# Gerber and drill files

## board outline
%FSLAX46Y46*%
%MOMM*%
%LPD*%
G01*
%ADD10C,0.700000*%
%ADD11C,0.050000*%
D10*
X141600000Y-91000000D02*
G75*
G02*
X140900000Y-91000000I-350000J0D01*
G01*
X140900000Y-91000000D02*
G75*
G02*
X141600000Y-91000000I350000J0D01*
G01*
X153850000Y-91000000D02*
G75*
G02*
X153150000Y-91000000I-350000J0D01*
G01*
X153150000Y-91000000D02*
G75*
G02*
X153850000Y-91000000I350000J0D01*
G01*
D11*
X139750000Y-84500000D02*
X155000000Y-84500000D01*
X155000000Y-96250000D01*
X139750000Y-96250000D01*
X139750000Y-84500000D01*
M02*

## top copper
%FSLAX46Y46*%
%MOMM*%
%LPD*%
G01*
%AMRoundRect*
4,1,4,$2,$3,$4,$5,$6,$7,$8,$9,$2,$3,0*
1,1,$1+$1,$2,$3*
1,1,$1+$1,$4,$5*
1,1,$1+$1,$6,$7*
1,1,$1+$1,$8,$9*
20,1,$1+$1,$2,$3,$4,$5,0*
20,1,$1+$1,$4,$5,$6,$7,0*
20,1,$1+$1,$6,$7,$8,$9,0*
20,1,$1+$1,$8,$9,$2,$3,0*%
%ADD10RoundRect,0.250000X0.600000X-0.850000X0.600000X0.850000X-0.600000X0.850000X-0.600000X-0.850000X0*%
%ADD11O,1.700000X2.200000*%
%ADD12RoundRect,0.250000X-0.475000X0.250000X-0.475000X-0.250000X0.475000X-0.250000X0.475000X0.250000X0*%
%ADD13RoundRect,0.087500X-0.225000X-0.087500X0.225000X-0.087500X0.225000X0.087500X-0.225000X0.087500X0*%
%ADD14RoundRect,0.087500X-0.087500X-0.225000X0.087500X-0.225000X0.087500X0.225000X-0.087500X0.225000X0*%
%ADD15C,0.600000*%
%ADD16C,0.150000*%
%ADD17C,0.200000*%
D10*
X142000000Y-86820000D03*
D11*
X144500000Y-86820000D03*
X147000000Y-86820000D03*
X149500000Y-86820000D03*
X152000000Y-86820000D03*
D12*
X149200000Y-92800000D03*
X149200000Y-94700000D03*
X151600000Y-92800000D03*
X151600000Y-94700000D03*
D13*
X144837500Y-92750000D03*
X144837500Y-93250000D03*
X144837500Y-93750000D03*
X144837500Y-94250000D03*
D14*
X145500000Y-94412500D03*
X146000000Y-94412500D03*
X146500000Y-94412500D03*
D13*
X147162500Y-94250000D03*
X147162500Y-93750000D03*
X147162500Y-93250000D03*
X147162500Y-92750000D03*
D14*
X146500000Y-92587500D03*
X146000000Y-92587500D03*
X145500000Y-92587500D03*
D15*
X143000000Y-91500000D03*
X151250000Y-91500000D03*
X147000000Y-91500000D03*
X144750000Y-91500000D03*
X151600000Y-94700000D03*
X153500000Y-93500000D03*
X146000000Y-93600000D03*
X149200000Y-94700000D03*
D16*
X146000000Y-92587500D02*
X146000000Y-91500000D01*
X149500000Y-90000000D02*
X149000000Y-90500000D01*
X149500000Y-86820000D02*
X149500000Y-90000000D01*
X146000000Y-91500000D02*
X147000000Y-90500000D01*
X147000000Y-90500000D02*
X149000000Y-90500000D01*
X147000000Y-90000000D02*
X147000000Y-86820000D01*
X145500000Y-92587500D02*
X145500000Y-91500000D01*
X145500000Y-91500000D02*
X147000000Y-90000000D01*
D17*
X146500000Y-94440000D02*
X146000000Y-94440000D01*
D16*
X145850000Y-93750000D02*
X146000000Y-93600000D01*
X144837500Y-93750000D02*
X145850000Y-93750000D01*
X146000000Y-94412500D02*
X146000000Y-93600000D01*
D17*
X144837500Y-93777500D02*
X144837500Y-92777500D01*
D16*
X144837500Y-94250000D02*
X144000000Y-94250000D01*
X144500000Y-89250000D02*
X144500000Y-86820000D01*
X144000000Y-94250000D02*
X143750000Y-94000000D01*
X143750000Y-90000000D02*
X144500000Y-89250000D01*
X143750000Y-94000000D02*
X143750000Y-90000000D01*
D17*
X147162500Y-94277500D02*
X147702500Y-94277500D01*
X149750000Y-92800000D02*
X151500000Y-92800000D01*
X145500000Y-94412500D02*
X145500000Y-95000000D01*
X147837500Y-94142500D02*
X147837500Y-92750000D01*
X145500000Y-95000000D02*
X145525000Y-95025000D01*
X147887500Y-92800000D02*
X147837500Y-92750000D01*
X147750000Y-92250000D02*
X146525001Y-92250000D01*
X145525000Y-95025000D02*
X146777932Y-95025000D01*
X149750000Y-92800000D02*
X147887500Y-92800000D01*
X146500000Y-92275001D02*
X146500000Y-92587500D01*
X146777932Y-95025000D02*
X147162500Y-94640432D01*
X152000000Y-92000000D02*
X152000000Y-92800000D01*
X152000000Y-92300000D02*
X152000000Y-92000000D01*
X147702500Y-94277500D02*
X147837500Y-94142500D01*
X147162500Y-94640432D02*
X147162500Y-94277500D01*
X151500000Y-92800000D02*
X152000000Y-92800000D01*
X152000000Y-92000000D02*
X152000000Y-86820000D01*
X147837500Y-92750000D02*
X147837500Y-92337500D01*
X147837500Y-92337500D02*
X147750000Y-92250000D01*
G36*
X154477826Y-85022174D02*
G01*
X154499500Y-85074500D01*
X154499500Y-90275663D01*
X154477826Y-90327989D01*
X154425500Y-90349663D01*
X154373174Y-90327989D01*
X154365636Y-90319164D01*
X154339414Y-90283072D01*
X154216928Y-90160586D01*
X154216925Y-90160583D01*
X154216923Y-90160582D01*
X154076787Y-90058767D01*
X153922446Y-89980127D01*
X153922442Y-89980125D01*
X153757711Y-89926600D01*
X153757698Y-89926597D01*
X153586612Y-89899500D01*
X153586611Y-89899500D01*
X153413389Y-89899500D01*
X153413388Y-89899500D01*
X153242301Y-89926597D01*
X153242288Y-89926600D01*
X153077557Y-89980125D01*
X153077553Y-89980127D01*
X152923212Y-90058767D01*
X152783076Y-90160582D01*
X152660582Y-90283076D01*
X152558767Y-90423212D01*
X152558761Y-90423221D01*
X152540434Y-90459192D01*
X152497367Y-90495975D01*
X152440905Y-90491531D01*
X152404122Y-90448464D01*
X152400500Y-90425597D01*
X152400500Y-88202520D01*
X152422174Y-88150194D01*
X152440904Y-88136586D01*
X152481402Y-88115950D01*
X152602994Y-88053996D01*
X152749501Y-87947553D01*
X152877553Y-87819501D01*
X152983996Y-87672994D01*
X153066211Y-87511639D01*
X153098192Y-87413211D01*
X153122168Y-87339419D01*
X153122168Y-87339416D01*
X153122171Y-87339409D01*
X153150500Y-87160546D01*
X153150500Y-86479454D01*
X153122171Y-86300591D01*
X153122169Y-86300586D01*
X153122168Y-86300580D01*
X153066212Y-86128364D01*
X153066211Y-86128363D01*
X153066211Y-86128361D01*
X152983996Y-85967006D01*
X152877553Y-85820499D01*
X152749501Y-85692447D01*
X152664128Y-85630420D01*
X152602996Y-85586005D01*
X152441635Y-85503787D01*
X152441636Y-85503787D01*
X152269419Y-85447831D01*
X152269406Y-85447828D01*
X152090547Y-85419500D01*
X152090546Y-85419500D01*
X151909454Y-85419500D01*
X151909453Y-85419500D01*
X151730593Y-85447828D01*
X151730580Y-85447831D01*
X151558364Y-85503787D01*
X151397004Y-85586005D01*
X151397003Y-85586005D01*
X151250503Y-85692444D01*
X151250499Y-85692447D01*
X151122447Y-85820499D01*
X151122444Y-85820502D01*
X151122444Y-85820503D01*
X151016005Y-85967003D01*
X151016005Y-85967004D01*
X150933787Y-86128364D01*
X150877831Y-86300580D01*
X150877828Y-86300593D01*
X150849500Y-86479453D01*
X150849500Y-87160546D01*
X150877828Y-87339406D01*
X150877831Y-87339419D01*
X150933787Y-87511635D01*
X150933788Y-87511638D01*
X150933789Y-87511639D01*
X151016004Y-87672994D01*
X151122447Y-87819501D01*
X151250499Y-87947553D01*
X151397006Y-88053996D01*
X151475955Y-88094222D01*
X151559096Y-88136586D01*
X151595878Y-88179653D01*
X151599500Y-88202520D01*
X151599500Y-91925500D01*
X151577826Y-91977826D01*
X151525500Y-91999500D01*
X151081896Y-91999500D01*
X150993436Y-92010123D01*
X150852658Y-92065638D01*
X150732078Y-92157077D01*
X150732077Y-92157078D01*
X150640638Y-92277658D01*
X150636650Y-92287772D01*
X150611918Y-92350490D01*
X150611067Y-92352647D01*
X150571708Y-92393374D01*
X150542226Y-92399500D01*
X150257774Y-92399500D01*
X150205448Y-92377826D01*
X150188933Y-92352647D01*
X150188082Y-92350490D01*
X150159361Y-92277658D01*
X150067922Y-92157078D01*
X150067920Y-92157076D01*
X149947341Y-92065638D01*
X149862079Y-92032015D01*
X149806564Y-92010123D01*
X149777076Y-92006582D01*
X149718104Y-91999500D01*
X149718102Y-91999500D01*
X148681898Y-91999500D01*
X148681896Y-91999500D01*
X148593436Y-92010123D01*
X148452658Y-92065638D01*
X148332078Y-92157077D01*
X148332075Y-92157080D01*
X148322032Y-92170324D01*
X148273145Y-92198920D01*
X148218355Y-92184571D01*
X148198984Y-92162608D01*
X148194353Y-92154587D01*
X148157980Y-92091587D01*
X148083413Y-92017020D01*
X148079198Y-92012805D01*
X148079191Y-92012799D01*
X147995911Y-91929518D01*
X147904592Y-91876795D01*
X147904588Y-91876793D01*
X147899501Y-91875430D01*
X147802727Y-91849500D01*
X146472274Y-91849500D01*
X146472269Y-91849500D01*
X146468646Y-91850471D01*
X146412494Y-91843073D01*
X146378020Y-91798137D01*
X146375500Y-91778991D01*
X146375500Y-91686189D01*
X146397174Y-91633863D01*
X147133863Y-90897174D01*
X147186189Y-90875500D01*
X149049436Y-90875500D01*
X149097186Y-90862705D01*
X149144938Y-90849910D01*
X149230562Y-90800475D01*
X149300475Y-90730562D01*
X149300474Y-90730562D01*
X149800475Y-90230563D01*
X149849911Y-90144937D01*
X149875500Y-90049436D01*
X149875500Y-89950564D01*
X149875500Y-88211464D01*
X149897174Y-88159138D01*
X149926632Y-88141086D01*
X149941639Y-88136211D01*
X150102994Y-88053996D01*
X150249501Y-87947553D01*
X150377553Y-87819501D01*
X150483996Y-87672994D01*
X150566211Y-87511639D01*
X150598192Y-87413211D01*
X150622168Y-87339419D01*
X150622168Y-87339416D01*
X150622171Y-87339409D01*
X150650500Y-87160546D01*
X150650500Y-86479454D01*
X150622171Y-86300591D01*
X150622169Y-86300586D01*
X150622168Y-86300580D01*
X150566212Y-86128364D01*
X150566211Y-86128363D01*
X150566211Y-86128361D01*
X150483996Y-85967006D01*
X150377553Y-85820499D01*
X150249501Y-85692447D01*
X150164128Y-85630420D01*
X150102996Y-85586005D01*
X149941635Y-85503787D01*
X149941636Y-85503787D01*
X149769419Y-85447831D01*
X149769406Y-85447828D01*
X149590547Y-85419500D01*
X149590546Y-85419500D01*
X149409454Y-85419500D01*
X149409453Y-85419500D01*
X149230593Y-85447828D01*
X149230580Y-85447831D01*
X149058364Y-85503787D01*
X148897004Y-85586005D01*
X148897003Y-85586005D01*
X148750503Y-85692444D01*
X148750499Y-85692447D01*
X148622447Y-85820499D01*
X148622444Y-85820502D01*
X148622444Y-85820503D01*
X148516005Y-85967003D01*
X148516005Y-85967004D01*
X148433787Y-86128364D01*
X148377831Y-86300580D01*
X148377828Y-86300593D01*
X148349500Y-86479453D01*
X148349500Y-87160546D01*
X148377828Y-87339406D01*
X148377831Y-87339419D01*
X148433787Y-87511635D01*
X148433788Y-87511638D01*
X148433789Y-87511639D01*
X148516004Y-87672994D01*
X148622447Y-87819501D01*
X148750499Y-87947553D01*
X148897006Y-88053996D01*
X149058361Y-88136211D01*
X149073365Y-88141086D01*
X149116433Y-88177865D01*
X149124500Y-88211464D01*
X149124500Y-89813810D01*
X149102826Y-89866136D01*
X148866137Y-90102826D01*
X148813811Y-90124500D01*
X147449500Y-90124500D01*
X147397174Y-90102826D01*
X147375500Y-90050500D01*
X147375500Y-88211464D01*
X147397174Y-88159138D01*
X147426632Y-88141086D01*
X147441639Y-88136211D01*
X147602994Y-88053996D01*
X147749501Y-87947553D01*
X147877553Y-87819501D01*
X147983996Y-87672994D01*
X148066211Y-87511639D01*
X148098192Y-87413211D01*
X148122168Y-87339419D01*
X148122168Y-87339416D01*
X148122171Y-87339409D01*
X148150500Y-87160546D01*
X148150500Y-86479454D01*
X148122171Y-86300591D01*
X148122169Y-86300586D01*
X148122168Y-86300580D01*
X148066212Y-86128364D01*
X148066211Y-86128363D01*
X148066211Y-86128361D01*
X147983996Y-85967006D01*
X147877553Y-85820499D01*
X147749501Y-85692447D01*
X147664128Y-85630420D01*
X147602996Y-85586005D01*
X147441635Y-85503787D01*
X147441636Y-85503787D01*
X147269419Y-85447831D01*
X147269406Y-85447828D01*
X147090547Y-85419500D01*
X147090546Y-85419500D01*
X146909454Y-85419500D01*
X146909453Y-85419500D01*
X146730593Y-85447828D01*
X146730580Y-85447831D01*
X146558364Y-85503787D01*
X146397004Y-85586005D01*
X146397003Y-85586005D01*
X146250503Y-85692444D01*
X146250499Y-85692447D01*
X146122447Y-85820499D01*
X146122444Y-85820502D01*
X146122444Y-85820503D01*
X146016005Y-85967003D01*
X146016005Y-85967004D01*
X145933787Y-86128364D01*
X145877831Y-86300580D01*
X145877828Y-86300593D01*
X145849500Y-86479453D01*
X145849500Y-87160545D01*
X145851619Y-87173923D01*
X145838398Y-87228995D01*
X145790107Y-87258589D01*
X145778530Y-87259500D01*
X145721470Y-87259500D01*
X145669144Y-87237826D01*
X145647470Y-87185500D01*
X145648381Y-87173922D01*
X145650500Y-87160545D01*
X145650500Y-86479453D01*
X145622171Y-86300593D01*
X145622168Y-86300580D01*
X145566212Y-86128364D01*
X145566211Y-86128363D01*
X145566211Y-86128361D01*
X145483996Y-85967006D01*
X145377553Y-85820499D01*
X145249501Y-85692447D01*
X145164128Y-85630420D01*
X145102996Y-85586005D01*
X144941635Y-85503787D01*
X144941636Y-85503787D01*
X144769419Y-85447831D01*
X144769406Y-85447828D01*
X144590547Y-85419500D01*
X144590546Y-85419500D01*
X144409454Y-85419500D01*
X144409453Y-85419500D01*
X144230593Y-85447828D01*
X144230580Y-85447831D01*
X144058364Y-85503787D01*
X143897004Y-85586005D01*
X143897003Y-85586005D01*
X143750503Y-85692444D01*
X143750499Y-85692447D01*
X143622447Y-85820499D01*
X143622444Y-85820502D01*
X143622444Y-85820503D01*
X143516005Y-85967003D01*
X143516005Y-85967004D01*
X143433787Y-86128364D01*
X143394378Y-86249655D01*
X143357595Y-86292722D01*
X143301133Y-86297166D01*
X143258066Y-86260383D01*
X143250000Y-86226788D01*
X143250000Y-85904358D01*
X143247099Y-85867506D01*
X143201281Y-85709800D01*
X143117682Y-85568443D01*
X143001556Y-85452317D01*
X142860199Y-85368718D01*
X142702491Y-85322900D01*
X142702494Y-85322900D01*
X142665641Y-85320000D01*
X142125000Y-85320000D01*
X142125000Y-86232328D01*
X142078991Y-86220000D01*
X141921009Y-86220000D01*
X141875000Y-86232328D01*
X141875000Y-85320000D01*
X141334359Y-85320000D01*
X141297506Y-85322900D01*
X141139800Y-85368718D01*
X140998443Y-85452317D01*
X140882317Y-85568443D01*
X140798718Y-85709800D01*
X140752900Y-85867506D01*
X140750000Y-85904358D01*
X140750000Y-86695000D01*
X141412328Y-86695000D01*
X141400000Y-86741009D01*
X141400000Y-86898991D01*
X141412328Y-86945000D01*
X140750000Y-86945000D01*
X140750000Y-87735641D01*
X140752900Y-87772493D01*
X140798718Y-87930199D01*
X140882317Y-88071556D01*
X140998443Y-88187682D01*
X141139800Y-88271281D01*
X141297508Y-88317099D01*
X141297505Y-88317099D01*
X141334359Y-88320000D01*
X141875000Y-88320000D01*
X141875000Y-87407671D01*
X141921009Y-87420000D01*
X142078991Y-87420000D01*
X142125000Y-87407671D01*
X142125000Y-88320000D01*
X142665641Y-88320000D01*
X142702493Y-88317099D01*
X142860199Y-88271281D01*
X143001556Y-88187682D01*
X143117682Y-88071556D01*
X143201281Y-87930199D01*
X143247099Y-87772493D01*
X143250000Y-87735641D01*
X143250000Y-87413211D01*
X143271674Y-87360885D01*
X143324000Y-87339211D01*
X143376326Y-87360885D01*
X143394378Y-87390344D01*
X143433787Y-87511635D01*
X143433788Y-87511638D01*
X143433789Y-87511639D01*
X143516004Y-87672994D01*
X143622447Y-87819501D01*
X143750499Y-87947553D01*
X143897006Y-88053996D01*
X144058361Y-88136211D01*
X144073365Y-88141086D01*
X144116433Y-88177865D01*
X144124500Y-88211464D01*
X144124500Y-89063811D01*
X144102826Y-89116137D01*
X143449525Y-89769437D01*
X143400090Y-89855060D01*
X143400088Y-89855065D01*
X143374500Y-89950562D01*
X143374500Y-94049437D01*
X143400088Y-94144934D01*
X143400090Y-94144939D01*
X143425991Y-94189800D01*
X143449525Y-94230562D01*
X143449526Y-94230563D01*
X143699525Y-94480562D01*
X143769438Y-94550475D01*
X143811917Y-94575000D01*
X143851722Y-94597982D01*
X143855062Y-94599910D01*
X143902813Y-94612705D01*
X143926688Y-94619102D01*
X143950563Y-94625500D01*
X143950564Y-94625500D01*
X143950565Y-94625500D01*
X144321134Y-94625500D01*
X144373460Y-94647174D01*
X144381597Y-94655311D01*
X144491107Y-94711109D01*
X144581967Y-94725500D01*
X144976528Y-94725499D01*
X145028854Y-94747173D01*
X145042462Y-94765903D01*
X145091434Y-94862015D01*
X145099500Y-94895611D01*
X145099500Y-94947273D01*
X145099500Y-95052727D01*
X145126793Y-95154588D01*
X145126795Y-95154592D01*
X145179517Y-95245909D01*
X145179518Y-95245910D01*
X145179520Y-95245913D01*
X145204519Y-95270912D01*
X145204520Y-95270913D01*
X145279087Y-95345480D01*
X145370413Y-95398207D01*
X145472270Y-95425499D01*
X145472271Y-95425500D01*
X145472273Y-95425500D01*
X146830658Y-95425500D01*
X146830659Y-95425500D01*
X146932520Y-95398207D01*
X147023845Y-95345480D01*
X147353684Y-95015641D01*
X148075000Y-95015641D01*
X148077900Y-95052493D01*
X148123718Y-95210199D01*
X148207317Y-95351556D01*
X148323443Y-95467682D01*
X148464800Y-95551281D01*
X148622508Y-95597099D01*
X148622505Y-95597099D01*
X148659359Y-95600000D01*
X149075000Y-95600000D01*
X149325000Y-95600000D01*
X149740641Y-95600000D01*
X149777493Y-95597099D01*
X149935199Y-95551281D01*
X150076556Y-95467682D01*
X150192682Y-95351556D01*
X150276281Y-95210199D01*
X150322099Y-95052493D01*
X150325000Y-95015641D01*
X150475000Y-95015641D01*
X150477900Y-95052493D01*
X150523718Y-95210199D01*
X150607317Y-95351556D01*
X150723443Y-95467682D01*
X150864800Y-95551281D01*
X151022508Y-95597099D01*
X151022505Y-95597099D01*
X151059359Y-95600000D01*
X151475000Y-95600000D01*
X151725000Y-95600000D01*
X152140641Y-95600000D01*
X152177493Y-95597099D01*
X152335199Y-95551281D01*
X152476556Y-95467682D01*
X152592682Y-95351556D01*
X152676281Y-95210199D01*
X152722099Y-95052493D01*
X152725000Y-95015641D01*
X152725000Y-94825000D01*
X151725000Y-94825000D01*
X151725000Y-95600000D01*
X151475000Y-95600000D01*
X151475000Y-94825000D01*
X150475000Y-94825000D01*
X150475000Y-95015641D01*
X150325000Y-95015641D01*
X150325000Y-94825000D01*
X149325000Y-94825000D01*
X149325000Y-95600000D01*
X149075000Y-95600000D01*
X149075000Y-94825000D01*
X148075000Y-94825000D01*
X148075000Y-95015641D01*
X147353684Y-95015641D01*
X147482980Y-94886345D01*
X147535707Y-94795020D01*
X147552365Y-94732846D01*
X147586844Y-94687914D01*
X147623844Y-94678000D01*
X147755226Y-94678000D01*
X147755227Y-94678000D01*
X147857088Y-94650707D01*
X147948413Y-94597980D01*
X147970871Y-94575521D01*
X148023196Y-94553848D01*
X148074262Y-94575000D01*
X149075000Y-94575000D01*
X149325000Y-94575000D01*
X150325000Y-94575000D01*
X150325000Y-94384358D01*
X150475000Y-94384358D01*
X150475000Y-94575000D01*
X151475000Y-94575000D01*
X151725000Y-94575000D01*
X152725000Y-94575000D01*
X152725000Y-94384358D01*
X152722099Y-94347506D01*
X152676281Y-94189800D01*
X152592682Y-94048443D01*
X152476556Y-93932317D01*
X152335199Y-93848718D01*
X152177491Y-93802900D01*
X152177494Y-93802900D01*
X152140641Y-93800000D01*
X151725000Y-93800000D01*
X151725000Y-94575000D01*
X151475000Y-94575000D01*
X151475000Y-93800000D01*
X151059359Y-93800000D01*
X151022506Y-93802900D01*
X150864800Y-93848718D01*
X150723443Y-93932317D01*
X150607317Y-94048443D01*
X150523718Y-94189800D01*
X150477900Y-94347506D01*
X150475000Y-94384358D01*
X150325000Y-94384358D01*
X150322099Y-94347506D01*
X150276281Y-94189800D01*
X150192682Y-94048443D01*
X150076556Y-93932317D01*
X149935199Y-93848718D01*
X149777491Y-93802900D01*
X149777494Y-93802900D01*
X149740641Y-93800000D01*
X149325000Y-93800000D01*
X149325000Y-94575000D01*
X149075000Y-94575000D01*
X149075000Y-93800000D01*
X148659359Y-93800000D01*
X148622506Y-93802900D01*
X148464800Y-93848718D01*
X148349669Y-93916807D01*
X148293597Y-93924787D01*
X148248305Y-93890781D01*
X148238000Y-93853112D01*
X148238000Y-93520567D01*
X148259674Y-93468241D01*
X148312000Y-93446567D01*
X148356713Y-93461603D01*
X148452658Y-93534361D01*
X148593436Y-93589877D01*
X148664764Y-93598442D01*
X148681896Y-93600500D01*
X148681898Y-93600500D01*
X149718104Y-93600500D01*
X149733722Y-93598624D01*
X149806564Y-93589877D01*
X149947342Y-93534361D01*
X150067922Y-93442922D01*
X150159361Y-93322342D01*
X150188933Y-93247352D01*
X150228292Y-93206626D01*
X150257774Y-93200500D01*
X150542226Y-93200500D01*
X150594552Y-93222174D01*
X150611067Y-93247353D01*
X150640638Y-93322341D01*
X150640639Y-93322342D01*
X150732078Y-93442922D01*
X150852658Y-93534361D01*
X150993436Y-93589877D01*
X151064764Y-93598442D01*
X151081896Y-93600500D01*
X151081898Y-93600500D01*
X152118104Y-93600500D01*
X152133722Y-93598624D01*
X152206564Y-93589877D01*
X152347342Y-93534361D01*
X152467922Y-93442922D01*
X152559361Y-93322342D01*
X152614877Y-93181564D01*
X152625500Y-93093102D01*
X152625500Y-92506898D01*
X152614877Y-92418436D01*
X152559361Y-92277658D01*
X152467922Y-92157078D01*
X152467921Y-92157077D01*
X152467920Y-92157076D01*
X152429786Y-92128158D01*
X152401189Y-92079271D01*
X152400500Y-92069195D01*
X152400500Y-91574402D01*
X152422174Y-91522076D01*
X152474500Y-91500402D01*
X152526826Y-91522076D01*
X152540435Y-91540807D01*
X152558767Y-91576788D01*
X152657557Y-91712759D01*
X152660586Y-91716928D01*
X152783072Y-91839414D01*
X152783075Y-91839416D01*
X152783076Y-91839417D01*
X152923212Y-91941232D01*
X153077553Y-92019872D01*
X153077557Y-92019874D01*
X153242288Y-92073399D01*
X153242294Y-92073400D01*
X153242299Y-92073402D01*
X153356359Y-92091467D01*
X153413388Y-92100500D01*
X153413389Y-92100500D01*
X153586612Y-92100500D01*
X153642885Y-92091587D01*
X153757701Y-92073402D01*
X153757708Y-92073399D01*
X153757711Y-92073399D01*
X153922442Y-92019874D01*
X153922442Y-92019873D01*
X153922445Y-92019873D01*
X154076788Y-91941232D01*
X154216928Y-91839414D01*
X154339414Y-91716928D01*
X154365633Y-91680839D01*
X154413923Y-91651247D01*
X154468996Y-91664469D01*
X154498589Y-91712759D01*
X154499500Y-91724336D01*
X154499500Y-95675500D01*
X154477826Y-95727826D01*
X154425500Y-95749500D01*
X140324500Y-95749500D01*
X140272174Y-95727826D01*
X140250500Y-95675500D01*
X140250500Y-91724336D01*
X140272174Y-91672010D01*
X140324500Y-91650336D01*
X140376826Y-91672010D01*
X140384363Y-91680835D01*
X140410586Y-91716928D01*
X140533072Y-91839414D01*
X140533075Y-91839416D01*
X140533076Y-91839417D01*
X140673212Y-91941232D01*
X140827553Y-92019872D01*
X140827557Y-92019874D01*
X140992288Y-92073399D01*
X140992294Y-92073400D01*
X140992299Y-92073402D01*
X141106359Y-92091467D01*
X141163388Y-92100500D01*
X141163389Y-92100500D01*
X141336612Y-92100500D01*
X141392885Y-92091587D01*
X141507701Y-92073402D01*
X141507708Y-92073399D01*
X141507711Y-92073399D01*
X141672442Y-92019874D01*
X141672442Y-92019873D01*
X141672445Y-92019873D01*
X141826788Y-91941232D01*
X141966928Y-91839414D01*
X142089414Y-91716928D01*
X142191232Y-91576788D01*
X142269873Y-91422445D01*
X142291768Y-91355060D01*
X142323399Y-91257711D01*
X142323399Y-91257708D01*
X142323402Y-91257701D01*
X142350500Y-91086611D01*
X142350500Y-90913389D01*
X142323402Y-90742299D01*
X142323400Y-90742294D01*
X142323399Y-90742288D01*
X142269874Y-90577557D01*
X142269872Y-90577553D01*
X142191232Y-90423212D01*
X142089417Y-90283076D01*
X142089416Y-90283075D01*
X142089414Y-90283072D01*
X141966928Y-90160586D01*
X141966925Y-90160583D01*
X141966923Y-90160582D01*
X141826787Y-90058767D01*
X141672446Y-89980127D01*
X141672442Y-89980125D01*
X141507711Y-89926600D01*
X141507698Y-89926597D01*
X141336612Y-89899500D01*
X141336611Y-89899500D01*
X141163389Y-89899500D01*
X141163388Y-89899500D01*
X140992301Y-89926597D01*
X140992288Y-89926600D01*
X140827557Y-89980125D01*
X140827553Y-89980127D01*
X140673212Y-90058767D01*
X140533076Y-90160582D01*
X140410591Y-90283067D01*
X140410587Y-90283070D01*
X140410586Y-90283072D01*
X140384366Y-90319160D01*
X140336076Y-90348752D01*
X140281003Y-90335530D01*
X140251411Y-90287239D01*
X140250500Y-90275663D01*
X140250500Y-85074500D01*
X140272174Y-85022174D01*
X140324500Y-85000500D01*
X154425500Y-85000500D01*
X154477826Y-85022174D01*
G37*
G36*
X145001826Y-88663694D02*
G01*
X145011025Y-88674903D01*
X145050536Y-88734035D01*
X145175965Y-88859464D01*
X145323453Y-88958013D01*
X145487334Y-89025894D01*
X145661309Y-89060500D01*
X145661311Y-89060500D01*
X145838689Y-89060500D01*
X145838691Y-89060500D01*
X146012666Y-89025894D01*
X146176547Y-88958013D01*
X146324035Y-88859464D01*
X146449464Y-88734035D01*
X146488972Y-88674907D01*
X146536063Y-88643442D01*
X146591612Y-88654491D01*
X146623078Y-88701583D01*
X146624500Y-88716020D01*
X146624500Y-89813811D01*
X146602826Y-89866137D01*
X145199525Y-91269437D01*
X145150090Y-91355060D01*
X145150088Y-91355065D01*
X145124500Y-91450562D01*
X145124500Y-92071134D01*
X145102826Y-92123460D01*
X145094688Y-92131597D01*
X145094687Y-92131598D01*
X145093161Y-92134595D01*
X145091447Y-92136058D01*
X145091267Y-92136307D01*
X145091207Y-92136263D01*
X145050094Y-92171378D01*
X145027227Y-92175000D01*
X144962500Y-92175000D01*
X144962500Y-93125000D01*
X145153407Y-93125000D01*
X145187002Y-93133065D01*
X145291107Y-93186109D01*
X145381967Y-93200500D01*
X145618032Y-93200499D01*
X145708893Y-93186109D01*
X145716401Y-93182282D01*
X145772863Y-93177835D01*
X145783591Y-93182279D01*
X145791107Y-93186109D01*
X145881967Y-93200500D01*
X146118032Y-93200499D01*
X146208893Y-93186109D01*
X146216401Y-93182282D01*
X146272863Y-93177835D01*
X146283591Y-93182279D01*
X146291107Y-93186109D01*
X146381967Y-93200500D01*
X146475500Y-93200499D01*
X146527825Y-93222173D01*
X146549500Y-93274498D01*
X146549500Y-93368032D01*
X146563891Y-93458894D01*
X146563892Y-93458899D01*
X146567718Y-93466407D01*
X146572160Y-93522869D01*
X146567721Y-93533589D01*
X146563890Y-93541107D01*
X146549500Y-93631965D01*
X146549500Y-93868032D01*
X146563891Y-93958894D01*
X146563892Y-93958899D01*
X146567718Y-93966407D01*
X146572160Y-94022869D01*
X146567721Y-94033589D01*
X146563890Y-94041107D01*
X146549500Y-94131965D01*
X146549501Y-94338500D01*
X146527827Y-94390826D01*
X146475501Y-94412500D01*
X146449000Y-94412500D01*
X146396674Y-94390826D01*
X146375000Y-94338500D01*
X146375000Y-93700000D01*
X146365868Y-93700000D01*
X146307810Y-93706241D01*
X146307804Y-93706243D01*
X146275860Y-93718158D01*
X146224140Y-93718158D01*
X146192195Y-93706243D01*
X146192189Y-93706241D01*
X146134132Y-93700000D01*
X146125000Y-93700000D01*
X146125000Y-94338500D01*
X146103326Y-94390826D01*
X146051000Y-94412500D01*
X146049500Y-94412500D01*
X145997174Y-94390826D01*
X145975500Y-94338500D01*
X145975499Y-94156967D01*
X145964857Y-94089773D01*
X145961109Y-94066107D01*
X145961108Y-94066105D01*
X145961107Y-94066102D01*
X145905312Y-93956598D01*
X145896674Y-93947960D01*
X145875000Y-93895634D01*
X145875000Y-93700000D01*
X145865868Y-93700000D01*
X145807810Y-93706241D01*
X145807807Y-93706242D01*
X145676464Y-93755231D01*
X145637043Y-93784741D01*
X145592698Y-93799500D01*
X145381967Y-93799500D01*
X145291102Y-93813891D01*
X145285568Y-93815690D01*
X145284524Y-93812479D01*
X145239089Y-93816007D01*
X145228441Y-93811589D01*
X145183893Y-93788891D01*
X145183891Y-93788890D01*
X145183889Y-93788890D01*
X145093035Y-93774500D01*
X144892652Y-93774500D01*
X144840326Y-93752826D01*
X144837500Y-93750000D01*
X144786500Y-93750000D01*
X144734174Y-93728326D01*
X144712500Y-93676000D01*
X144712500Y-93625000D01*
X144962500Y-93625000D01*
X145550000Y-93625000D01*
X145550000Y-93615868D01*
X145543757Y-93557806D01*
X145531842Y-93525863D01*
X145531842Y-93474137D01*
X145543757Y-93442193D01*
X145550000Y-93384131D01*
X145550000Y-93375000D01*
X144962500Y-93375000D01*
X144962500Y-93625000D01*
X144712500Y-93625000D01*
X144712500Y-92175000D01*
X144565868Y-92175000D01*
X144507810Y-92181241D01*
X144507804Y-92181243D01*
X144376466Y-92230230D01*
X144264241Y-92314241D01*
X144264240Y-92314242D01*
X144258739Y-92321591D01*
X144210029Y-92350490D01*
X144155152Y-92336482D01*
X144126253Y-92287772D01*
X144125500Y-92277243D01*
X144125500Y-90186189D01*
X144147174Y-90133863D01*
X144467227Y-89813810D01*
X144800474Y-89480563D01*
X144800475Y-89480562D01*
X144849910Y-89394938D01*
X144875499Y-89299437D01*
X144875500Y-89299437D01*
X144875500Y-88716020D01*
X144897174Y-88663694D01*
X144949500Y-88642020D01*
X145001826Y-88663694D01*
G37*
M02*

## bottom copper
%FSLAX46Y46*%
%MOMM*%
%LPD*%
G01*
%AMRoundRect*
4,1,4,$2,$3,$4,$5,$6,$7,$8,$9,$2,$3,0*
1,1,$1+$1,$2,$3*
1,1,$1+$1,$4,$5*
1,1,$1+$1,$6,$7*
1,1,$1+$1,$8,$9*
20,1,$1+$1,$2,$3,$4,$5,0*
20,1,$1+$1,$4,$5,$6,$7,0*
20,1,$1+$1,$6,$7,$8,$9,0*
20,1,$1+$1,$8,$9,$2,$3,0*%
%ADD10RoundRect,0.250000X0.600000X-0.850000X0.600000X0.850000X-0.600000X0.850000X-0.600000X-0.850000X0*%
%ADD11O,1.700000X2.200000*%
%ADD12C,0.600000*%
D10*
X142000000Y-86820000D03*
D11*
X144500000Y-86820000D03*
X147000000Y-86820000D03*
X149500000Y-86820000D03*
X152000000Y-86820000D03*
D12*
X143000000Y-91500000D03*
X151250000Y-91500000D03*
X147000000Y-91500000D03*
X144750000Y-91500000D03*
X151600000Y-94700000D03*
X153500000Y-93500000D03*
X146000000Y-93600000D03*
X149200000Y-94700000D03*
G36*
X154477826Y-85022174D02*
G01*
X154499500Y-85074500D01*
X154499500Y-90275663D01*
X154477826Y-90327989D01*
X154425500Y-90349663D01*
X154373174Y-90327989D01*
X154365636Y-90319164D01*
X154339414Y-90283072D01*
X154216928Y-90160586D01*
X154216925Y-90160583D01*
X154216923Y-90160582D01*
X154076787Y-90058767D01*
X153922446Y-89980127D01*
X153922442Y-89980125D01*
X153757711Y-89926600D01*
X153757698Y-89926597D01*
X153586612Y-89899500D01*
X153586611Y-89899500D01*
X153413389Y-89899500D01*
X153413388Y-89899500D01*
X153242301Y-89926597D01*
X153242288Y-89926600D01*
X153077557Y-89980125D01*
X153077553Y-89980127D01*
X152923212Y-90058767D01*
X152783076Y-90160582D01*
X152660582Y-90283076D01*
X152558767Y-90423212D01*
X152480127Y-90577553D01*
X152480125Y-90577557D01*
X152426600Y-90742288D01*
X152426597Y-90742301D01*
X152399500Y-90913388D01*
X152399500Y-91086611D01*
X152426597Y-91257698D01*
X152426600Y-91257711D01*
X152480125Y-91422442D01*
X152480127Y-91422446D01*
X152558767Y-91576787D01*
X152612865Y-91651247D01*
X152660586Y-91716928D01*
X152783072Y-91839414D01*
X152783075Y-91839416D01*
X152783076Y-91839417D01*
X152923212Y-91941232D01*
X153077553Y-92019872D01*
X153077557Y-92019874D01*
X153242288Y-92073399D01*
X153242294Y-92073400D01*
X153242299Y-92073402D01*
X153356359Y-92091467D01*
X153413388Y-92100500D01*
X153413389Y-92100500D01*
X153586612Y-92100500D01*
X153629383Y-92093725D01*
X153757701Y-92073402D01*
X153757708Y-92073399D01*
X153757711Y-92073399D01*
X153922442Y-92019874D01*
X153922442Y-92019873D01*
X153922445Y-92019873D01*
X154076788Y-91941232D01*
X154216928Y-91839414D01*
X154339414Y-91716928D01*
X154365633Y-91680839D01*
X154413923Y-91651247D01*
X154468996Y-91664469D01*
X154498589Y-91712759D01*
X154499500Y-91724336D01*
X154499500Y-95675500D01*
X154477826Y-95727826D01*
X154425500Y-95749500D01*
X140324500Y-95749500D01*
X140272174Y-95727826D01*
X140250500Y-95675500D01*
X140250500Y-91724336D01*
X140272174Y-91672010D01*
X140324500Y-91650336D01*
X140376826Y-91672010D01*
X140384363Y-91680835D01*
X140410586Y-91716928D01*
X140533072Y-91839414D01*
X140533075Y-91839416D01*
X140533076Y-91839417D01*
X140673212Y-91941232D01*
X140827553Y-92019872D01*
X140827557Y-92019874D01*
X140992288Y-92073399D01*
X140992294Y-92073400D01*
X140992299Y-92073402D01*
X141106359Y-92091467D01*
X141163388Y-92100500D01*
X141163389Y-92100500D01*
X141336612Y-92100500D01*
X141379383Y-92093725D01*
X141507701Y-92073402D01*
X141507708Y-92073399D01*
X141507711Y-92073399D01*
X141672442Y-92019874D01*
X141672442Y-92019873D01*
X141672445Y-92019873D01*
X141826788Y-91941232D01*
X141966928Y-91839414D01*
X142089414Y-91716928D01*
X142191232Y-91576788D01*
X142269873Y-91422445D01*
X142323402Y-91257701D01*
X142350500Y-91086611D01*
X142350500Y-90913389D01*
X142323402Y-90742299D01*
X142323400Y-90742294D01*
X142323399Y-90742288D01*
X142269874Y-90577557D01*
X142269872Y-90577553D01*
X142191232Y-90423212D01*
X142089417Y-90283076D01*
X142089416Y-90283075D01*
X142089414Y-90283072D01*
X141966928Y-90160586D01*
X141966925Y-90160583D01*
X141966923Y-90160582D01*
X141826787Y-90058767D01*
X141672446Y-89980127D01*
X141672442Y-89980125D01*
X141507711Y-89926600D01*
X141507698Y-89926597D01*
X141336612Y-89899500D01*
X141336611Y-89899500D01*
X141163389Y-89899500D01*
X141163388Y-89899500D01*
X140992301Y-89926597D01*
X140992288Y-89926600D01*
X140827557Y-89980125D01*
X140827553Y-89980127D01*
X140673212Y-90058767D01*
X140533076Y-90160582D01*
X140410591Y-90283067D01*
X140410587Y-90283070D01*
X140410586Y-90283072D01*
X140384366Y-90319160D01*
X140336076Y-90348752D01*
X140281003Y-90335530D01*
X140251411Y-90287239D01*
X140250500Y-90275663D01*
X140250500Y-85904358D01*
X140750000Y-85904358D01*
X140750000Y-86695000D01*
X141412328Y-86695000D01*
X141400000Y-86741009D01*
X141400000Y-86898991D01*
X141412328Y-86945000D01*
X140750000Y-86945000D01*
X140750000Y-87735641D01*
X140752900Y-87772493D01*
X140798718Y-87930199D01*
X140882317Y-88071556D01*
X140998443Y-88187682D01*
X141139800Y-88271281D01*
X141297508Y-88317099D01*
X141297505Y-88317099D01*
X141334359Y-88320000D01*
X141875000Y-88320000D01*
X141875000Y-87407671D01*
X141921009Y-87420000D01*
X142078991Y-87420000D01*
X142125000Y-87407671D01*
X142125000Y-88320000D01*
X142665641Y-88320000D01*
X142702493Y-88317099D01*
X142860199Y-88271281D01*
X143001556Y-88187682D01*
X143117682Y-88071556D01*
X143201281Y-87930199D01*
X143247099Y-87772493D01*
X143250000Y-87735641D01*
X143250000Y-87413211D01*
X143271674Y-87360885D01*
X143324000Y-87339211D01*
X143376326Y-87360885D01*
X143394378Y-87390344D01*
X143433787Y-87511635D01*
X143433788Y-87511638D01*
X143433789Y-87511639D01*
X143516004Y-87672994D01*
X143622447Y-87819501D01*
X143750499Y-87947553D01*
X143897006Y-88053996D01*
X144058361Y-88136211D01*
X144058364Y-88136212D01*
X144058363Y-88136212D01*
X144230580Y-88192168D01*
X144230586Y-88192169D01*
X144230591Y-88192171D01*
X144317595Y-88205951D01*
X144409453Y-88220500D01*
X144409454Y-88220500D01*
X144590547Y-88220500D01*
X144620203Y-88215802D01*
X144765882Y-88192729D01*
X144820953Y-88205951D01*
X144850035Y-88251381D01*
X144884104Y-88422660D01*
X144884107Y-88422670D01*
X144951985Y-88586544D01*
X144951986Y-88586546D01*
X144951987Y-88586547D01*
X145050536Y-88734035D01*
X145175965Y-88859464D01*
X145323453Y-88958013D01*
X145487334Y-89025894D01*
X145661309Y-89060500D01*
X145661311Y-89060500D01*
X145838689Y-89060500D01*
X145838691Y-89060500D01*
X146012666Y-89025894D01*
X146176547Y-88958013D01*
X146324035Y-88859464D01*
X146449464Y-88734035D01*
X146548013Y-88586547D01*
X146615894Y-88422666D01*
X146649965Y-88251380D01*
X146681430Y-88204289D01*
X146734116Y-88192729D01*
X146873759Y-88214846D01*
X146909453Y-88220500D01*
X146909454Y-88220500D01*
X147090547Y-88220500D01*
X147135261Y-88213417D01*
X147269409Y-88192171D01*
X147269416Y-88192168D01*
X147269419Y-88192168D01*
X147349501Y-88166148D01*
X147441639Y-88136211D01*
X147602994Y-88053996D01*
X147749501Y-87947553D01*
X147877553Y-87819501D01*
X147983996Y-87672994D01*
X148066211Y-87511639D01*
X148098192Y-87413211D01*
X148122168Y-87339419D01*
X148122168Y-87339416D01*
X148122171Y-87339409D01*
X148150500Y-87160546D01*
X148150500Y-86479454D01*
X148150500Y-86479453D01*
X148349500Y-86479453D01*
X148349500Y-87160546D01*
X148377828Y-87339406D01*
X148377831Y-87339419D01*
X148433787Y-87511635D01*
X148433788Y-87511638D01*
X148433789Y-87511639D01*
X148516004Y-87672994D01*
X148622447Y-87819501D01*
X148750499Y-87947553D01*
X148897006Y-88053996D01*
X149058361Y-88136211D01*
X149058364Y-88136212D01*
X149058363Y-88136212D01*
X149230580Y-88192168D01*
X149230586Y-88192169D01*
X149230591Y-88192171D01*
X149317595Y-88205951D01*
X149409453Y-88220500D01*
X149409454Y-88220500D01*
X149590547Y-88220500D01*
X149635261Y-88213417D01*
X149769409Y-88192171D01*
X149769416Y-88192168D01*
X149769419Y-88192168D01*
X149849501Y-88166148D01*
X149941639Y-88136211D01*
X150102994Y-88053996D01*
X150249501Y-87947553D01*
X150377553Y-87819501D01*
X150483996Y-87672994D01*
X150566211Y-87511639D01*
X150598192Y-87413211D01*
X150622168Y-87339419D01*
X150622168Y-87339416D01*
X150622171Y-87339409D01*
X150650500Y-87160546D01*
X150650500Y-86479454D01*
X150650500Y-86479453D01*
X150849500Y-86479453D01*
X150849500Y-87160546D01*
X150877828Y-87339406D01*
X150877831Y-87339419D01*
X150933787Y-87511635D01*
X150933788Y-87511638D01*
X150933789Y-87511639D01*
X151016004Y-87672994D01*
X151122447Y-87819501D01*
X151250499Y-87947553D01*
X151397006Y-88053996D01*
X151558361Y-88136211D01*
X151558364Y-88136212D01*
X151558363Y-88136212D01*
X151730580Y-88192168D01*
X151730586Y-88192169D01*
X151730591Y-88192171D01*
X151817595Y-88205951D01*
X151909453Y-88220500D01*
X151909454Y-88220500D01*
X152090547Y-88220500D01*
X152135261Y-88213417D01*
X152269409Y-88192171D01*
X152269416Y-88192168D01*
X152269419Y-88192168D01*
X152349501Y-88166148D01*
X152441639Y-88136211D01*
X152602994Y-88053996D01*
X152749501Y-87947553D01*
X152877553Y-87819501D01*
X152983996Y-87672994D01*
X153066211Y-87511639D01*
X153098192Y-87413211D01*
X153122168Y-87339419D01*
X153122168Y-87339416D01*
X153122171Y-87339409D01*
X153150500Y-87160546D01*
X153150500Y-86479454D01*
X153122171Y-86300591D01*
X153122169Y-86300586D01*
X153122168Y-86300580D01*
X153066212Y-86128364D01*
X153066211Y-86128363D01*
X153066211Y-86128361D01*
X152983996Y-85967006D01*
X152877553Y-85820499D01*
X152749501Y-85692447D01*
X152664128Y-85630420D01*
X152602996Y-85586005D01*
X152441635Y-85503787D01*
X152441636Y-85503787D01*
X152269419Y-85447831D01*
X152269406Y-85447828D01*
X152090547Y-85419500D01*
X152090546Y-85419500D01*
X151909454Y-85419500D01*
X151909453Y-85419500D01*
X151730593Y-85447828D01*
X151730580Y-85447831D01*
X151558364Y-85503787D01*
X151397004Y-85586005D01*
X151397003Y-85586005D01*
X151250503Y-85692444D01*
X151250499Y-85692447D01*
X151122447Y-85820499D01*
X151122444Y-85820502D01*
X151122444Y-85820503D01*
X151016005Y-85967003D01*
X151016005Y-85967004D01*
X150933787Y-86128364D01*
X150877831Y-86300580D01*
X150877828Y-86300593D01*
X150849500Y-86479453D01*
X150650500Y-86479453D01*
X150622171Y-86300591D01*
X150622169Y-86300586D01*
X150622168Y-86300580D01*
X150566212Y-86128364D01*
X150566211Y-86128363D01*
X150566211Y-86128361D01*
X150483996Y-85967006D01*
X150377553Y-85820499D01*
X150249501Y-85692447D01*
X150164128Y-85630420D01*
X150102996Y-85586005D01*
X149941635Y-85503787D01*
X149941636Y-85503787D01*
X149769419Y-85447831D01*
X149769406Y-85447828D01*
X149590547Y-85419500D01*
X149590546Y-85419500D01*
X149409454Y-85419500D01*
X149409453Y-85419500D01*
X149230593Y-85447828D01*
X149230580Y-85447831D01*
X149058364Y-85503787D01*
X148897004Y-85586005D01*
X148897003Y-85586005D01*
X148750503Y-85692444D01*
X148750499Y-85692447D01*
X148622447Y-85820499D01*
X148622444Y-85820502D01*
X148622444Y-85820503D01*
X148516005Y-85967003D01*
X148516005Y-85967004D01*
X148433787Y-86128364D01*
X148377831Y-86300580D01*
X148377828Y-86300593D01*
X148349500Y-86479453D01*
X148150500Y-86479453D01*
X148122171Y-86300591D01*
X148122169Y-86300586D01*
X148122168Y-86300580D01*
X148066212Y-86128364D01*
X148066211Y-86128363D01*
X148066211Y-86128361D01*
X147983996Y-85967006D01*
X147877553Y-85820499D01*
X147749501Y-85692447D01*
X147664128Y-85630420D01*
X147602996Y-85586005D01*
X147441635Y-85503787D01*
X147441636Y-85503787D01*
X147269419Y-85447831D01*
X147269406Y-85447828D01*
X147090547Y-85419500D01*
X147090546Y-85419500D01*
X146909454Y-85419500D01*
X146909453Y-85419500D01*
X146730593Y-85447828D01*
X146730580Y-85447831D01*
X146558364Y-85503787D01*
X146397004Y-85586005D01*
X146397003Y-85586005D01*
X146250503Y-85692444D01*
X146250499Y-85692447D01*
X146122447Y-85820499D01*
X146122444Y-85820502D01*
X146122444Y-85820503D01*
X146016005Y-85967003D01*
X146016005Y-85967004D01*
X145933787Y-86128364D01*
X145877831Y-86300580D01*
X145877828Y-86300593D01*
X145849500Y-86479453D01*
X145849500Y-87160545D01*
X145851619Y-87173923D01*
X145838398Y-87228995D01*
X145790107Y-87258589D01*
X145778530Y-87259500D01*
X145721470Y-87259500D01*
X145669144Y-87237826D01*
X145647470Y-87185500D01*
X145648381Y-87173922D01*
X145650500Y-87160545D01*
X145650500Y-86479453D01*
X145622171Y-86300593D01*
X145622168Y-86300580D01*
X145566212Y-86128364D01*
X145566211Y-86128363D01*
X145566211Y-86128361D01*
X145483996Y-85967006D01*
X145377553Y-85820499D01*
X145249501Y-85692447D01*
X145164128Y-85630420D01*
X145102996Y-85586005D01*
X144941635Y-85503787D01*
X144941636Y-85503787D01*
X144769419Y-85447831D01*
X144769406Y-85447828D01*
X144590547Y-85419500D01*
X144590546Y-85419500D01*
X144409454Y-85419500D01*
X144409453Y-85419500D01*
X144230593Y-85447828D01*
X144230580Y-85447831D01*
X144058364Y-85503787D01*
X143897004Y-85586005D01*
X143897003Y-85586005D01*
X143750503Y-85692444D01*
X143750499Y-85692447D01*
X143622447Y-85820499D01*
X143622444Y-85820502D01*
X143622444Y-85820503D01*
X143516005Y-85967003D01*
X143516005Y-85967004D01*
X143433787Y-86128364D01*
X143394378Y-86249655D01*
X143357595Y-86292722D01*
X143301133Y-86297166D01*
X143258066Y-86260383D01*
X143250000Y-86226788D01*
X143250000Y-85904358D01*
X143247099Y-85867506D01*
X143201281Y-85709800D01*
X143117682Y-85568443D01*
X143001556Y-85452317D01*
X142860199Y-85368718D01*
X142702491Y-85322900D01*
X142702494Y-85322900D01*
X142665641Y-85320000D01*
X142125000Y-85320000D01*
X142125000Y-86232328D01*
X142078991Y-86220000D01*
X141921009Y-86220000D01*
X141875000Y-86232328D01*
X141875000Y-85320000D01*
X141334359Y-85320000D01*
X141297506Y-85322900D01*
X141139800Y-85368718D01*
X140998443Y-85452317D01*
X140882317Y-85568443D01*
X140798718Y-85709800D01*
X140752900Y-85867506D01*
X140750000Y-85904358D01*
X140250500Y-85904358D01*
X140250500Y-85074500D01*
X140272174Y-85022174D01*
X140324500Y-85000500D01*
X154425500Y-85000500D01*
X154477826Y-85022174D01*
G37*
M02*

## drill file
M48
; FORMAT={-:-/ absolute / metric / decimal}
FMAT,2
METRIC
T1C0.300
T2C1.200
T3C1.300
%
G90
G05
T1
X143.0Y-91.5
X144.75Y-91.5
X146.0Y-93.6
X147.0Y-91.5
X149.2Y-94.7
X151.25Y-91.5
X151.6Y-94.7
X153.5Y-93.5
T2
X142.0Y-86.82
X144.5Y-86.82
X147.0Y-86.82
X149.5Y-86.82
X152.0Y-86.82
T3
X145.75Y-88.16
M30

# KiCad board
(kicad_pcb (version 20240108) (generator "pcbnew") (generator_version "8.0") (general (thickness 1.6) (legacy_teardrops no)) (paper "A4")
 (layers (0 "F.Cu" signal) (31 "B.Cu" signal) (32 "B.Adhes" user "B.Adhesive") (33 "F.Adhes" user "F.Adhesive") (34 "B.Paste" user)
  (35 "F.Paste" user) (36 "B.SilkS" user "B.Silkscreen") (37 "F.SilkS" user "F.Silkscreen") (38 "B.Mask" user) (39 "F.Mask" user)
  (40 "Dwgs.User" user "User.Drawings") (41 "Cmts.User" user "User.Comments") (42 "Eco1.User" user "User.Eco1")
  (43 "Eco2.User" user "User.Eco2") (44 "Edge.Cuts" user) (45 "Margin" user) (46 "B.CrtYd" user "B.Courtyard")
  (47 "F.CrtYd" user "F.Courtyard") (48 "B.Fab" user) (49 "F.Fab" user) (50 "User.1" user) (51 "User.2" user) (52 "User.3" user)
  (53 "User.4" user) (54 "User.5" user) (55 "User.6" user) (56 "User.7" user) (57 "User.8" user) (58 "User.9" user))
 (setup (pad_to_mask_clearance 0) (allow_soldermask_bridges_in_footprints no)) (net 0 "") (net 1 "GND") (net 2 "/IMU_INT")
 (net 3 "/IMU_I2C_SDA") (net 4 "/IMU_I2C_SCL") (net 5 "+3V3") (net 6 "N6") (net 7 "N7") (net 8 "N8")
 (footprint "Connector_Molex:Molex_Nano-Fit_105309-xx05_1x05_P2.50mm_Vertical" (layer "F.Cu") (at 142 86.82 90)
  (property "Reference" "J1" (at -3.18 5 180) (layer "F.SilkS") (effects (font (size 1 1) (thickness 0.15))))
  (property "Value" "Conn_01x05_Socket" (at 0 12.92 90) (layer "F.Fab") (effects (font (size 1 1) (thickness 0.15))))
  (pad "" np_thru_hole circle (at -1.34 3.75 90) (size 1.3 1.3) (drill 1.3) (layers "*.Cu" "*.Mask"))
  (pad "1" thru_hole roundrect (at 0 0 90) (size 2.2 1.7) (drill 1.2) (layers "*.Cu" "*.Mask") (remove_unused_layers no)
   (roundrect_rratio 0.147059) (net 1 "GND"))
  (pad "2" thru_hole oval (at 0 2.5 90) (size 2.2 1.7) (drill 1.2) (layers "*.Cu" "*.Mask") (remove_unused_layers no) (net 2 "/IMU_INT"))
  (pad "3" thru_hole oval (at 0 5 90) (size 2.2 1.7) (drill 1.2) (layers "*.Cu" "*.Mask") (remove_unused_layers no) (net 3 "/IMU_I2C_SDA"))
  (pad "4" thru_hole oval (at 0 7.5 90) (size 2.2 1.7) (drill 1.2) (layers "*.Cu" "*.Mask") (remove_unused_layers no) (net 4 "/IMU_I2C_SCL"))
  (pad "5" thru_hole oval (at 0 10 90) (size 2.2 1.7) (drill 1.2) (layers "*.Cu" "*.Mask") (remove_unused_layers no) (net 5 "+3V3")))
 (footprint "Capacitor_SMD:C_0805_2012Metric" (layer "F.Cu") (at 149.2 93.75 -90)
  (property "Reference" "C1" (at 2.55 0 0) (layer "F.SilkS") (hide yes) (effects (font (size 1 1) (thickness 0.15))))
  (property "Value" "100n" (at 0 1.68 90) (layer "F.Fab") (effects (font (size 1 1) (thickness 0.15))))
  (pad "1" smd roundrect (at -0.95 0 270) (size 1 1.45) (layers "F.Cu" "F.Paste" "F.Mask") (roundrect_rratio 0.25) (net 5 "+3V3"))
  (pad "2" smd roundrect (at 0.95 0 270) (size 1 1.45) (layers "F.Cu" "F.Paste" "F.Mask") (roundrect_rratio 0.25) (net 1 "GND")))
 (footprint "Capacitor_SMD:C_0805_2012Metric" (layer "F.Cu") (at 151.6 93.75 -90)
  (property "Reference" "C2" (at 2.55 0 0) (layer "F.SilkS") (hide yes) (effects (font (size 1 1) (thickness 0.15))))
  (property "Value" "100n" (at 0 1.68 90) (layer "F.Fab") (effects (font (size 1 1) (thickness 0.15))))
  (pad "1" smd roundrect (at -0.95 0 270) (size 1 1.45) (layers "F.Cu" "F.Paste" "F.Mask") (roundrect_rratio 0.25) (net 5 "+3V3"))
  (pad "2" smd roundrect (at 0.95 0 270) (size 1 1.45) (layers "F.Cu" "F.Paste" "F.Mask") (roundrect_rratio 0.25) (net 1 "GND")))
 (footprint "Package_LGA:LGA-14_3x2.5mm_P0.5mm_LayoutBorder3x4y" (layer "F.Cu") (at 146 93.5)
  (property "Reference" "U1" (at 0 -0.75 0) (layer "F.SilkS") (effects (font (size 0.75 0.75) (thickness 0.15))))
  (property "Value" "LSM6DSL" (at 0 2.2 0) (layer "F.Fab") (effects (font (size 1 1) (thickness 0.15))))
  (pad "1" smd roundrect (at -1.1625 -0.75) (size 0.625 0.35) (layers "F.Cu" "F.Paste" "F.Mask") (roundrect_rratio 0.25) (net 1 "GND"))
  (pad "2" smd roundrect (at -1.1625 -0.25) (size 0.625 0.35) (layers "F.Cu" "F.Paste" "F.Mask") (roundrect_rratio 0.25) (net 1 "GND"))
  (pad "3" smd roundrect (at -1.1625 0.25) (size 0.625 0.35) (layers "F.Cu" "F.Paste" "F.Mask") (roundrect_rratio 0.25) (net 1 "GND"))
  (pad "4" smd roundrect (at -1.1625 0.75) (size 0.625 0.35) (layers "F.Cu" "F.Paste" "F.Mask") (roundrect_rratio 0.25) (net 2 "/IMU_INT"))
  (pad "5" smd roundrect (at -0.5 0.9125) (size 0.35 0.625) (layers "F.Cu" "F.Paste" "F.Mask") (roundrect_rratio 0.25) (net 5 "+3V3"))
  (pad "6" smd roundrect (at 0 0.9125) (size 0.35 0.625) (layers "F.Cu" "F.Paste" "F.Mask") (roundrect_rratio 0.25) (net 1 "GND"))
  (pad "7" smd roundrect (at 0.5 0.9125) (size 0.35 0.625) (layers "F.Cu" "F.Paste" "F.Mask") (roundrect_rratio 0.25) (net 1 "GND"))
  (pad "8" smd roundrect (at 1.1625 0.75) (size 0.625 0.35) (layers "F.Cu" "F.Paste" "F.Mask") (roundrect_rratio 0.25) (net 5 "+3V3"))
  (pad "9" smd roundrect (at 1.1625 0.25) (size 0.625 0.35) (layers "F.Cu" "F.Paste" "F.Mask") (roundrect_rratio 0.25) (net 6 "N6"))
  (pad "10" smd roundrect (at 1.1625 -0.25) (size 0.625 0.35) (layers "F.Cu" "F.Paste" "F.Mask") (roundrect_rratio 0.25) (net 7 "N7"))
  (pad "11" smd roundrect (at 1.1625 -0.75) (size 0.625 0.35) (layers "F.Cu" "F.Paste" "F.Mask") (roundrect_rratio 0.25) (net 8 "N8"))
  (pad "12" smd roundrect (at 0.5 -0.9125) (size 0.35 0.625) (layers "F.Cu" "F.Paste" "F.Mask") (roundrect_rratio 0.25) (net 5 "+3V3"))
  (pad "13" smd roundrect (at 0 -0.9125) (size 0.35 0.625) (layers "F.Cu" "F.Paste" "F.Mask") (roundrect_rratio 0.25) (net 4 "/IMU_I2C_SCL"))
  (pad "14" smd roundrect (at -0.5 -0.9125) (size 0.35 0.625) (layers "F.Cu" "F.Paste" "F.Mask") (roundrect_rratio 0.25)
   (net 3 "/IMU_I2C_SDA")))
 (gr_circle (center 141.25 91) (end 141.85 91) (stroke (width 0.2) (type solid)) (fill solid) (layer "Edge.Cuts"))
 (gr_circle (center 153.5 91) (end 154.1 91) (stroke (width 0.2) (type solid)) (fill solid) (layer "Edge.Cuts"))
 (gr_rect (start 139.75 84.5) (end 155 96.25) (stroke (width 0.05) (type default)) (fill none) (layer "Edge.Cuts"))
 (segment (start 146 92.5875) (end 146 91.5) (width 0.15) (layer "F.Cu") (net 4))
 (segment (start 149.5 90) (end 149 90.5) (width 0.15) (layer "F.Cu") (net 4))
 (segment (start 149.5 86.82) (end 149.5 90) (width 0.15) (layer "F.Cu") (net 4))
 (segment (start 146 91.5) (end 147 90.5) (width 0.15) (layer "F.Cu") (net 4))
 (segment (start 147 90.5) (end 149 90.5) (width 0.15) (layer "F.Cu") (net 4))
 (segment (start 147 90) (end 147 86.82) (width 0.15) (layer "F.Cu") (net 3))
 (segment (start 145.5 92.5875) (end 145.5 91.5) (width 0.15) (layer "F.Cu") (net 3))
 (segment (start 145.5 91.5) (end 147 90) (width 0.15) (layer "F.Cu") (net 3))
 (segment (start 146.5 94.44) (end 146 94.44) (width 0.2) (layer "F.Cu") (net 1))
 (segment (start 145.85 93.75) (end 146 93.6) (width 0.15) (layer "F.Cu") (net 1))
 (segment (start 144.8375 93.75) (end 145.85 93.75) (width 0.15) (layer "F.Cu") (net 1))
 (segment (start 146 94.4125) (end 146 93.6) (width 0.15) (layer "F.Cu") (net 1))
 (segment (start 144.8375 93.7775) (end 144.8375 92.7775) (width 0.2) (layer "F.Cu") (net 1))
 (via (at 143 91.5) (size 0.6) (drill 0.3) (layers "F.Cu" "B.Cu") (free yes) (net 1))
 (via (at 151.25 91.5) (size 0.6) (drill 0.3) (layers "F.Cu" "B.Cu") (free yes) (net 1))
 (via (at 147 91.5) (size 0.6) (drill 0.3) (layers "F.Cu" "B.Cu") (free yes) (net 1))
 (via (at 144.75 91.5) (size 0.6) (drill 0.3) (layers "F.Cu" "B.Cu") (free yes) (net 1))
 (via (at 151.6 94.7) (size 0.6) (drill 0.3) (layers "F.Cu" "B.Cu") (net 1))
 (via (at 153.5 93.5) (size 0.6) (drill 0.3) (layers "F.Cu" "B.Cu") (free yes) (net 1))
 (via (at 146 93.6) (size 0.6) (drill 0.3) (layers "F.Cu" "B.Cu") (free yes) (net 1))
 (via (at 149.2 94.7) (size 0.6) (drill 0.3) (layers "F.Cu" "B.Cu") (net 1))
 (segment (start 144.8375 94.25) (end 144 94.25) (width 0.15) (layer "F.Cu") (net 2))
 (segment (start 144.5 89.25) (end 144.5 86.82) (width 0.15) (layer "F.Cu") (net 2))
 (segment (start 144 94.25) (end 143.75 94) (width 0.15) (layer "F.Cu") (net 2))
 (segment (start 143.75 90) (end 144.5 89.25) (width 0.15) (layer "F.Cu") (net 2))
 (segment (start 143.75 94) (end 143.75 90) (width 0.15) (layer "F.Cu") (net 2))
 (segment (start 147.1625 94.2775) (end 147.7025 94.2775) (width 0.2) (layer "F.Cu") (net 5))
 (segment (start 149.75 92.8) (end 151.5 92.8) (width 0.2) (layer "F.Cu") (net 5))
 (segment (start 145.5 94.4125) (end 145.5 95) (width 0.2) (layer "F.Cu") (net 5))
 (segment (start 147.8375 94.1425) (end 147.8375 92.75) (width 0.2) (layer "F.Cu") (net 5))
 (segment (start 145.5 95) (end 145.525 95.025) (width 0.2) (layer "F.Cu") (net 5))
 (segment (start 147.8875 92.8) (end 147.8375 92.75) (width 0.2) (layer "F.Cu") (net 5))
 (segment (start 147.75 92.25) (end 146.525001 92.25) (width 0.2) (layer "F.Cu") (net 5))
 (segment (start 145.525 95.025) (end 146.777932 95.025) (width 0.2) (layer "F.Cu") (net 5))
 (segment (start 149.75 92.8) (end 147.8875 92.8) (width 0.2) (layer "F.Cu") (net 5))
 (segment (start 146.5 92.275001) (end 146.5 92.5875) (width 0.2) (layer "F.Cu") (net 5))
 (segment (start 146.777932 95.025) (end 147.1625 94.640432) (width 0.2) (layer "F.Cu") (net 5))
 (segment (start 152 92) (end 152 92.8) (width 0.2) (layer "F.Cu") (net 5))
 (segment (start 152 92.3) (end 152 92) (width 0.2) (layer "F.Cu") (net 5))
 (segment (start 147.7025 94.2775) (end 147.8375 94.1425) (width 0.2) (layer "F.Cu") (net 5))
 (segment (start 147.1625 94.640432) (end 147.1625 94.2775) (width 0.2) (layer "F.Cu") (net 5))
 (segment (start 151.5 92.8) (end 152 92.8) (width 0.2) (layer "F.Cu") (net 5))
 (segment (start 152 92) (end 152 86.82) (width 0.2) (layer "F.Cu") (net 5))
 (segment (start 147.8375 92.75) (end 147.8375 92.3375) (width 0.2) (layer "F.Cu") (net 5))
 (segment (start 147.8375 92.3375) (end 147.75 92.25) (width 0.2) (layer "F.Cu") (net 5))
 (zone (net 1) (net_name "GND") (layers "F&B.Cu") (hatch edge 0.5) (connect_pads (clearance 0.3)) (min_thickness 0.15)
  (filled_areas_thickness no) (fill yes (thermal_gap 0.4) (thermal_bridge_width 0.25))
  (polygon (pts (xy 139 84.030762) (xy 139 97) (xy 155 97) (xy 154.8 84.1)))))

